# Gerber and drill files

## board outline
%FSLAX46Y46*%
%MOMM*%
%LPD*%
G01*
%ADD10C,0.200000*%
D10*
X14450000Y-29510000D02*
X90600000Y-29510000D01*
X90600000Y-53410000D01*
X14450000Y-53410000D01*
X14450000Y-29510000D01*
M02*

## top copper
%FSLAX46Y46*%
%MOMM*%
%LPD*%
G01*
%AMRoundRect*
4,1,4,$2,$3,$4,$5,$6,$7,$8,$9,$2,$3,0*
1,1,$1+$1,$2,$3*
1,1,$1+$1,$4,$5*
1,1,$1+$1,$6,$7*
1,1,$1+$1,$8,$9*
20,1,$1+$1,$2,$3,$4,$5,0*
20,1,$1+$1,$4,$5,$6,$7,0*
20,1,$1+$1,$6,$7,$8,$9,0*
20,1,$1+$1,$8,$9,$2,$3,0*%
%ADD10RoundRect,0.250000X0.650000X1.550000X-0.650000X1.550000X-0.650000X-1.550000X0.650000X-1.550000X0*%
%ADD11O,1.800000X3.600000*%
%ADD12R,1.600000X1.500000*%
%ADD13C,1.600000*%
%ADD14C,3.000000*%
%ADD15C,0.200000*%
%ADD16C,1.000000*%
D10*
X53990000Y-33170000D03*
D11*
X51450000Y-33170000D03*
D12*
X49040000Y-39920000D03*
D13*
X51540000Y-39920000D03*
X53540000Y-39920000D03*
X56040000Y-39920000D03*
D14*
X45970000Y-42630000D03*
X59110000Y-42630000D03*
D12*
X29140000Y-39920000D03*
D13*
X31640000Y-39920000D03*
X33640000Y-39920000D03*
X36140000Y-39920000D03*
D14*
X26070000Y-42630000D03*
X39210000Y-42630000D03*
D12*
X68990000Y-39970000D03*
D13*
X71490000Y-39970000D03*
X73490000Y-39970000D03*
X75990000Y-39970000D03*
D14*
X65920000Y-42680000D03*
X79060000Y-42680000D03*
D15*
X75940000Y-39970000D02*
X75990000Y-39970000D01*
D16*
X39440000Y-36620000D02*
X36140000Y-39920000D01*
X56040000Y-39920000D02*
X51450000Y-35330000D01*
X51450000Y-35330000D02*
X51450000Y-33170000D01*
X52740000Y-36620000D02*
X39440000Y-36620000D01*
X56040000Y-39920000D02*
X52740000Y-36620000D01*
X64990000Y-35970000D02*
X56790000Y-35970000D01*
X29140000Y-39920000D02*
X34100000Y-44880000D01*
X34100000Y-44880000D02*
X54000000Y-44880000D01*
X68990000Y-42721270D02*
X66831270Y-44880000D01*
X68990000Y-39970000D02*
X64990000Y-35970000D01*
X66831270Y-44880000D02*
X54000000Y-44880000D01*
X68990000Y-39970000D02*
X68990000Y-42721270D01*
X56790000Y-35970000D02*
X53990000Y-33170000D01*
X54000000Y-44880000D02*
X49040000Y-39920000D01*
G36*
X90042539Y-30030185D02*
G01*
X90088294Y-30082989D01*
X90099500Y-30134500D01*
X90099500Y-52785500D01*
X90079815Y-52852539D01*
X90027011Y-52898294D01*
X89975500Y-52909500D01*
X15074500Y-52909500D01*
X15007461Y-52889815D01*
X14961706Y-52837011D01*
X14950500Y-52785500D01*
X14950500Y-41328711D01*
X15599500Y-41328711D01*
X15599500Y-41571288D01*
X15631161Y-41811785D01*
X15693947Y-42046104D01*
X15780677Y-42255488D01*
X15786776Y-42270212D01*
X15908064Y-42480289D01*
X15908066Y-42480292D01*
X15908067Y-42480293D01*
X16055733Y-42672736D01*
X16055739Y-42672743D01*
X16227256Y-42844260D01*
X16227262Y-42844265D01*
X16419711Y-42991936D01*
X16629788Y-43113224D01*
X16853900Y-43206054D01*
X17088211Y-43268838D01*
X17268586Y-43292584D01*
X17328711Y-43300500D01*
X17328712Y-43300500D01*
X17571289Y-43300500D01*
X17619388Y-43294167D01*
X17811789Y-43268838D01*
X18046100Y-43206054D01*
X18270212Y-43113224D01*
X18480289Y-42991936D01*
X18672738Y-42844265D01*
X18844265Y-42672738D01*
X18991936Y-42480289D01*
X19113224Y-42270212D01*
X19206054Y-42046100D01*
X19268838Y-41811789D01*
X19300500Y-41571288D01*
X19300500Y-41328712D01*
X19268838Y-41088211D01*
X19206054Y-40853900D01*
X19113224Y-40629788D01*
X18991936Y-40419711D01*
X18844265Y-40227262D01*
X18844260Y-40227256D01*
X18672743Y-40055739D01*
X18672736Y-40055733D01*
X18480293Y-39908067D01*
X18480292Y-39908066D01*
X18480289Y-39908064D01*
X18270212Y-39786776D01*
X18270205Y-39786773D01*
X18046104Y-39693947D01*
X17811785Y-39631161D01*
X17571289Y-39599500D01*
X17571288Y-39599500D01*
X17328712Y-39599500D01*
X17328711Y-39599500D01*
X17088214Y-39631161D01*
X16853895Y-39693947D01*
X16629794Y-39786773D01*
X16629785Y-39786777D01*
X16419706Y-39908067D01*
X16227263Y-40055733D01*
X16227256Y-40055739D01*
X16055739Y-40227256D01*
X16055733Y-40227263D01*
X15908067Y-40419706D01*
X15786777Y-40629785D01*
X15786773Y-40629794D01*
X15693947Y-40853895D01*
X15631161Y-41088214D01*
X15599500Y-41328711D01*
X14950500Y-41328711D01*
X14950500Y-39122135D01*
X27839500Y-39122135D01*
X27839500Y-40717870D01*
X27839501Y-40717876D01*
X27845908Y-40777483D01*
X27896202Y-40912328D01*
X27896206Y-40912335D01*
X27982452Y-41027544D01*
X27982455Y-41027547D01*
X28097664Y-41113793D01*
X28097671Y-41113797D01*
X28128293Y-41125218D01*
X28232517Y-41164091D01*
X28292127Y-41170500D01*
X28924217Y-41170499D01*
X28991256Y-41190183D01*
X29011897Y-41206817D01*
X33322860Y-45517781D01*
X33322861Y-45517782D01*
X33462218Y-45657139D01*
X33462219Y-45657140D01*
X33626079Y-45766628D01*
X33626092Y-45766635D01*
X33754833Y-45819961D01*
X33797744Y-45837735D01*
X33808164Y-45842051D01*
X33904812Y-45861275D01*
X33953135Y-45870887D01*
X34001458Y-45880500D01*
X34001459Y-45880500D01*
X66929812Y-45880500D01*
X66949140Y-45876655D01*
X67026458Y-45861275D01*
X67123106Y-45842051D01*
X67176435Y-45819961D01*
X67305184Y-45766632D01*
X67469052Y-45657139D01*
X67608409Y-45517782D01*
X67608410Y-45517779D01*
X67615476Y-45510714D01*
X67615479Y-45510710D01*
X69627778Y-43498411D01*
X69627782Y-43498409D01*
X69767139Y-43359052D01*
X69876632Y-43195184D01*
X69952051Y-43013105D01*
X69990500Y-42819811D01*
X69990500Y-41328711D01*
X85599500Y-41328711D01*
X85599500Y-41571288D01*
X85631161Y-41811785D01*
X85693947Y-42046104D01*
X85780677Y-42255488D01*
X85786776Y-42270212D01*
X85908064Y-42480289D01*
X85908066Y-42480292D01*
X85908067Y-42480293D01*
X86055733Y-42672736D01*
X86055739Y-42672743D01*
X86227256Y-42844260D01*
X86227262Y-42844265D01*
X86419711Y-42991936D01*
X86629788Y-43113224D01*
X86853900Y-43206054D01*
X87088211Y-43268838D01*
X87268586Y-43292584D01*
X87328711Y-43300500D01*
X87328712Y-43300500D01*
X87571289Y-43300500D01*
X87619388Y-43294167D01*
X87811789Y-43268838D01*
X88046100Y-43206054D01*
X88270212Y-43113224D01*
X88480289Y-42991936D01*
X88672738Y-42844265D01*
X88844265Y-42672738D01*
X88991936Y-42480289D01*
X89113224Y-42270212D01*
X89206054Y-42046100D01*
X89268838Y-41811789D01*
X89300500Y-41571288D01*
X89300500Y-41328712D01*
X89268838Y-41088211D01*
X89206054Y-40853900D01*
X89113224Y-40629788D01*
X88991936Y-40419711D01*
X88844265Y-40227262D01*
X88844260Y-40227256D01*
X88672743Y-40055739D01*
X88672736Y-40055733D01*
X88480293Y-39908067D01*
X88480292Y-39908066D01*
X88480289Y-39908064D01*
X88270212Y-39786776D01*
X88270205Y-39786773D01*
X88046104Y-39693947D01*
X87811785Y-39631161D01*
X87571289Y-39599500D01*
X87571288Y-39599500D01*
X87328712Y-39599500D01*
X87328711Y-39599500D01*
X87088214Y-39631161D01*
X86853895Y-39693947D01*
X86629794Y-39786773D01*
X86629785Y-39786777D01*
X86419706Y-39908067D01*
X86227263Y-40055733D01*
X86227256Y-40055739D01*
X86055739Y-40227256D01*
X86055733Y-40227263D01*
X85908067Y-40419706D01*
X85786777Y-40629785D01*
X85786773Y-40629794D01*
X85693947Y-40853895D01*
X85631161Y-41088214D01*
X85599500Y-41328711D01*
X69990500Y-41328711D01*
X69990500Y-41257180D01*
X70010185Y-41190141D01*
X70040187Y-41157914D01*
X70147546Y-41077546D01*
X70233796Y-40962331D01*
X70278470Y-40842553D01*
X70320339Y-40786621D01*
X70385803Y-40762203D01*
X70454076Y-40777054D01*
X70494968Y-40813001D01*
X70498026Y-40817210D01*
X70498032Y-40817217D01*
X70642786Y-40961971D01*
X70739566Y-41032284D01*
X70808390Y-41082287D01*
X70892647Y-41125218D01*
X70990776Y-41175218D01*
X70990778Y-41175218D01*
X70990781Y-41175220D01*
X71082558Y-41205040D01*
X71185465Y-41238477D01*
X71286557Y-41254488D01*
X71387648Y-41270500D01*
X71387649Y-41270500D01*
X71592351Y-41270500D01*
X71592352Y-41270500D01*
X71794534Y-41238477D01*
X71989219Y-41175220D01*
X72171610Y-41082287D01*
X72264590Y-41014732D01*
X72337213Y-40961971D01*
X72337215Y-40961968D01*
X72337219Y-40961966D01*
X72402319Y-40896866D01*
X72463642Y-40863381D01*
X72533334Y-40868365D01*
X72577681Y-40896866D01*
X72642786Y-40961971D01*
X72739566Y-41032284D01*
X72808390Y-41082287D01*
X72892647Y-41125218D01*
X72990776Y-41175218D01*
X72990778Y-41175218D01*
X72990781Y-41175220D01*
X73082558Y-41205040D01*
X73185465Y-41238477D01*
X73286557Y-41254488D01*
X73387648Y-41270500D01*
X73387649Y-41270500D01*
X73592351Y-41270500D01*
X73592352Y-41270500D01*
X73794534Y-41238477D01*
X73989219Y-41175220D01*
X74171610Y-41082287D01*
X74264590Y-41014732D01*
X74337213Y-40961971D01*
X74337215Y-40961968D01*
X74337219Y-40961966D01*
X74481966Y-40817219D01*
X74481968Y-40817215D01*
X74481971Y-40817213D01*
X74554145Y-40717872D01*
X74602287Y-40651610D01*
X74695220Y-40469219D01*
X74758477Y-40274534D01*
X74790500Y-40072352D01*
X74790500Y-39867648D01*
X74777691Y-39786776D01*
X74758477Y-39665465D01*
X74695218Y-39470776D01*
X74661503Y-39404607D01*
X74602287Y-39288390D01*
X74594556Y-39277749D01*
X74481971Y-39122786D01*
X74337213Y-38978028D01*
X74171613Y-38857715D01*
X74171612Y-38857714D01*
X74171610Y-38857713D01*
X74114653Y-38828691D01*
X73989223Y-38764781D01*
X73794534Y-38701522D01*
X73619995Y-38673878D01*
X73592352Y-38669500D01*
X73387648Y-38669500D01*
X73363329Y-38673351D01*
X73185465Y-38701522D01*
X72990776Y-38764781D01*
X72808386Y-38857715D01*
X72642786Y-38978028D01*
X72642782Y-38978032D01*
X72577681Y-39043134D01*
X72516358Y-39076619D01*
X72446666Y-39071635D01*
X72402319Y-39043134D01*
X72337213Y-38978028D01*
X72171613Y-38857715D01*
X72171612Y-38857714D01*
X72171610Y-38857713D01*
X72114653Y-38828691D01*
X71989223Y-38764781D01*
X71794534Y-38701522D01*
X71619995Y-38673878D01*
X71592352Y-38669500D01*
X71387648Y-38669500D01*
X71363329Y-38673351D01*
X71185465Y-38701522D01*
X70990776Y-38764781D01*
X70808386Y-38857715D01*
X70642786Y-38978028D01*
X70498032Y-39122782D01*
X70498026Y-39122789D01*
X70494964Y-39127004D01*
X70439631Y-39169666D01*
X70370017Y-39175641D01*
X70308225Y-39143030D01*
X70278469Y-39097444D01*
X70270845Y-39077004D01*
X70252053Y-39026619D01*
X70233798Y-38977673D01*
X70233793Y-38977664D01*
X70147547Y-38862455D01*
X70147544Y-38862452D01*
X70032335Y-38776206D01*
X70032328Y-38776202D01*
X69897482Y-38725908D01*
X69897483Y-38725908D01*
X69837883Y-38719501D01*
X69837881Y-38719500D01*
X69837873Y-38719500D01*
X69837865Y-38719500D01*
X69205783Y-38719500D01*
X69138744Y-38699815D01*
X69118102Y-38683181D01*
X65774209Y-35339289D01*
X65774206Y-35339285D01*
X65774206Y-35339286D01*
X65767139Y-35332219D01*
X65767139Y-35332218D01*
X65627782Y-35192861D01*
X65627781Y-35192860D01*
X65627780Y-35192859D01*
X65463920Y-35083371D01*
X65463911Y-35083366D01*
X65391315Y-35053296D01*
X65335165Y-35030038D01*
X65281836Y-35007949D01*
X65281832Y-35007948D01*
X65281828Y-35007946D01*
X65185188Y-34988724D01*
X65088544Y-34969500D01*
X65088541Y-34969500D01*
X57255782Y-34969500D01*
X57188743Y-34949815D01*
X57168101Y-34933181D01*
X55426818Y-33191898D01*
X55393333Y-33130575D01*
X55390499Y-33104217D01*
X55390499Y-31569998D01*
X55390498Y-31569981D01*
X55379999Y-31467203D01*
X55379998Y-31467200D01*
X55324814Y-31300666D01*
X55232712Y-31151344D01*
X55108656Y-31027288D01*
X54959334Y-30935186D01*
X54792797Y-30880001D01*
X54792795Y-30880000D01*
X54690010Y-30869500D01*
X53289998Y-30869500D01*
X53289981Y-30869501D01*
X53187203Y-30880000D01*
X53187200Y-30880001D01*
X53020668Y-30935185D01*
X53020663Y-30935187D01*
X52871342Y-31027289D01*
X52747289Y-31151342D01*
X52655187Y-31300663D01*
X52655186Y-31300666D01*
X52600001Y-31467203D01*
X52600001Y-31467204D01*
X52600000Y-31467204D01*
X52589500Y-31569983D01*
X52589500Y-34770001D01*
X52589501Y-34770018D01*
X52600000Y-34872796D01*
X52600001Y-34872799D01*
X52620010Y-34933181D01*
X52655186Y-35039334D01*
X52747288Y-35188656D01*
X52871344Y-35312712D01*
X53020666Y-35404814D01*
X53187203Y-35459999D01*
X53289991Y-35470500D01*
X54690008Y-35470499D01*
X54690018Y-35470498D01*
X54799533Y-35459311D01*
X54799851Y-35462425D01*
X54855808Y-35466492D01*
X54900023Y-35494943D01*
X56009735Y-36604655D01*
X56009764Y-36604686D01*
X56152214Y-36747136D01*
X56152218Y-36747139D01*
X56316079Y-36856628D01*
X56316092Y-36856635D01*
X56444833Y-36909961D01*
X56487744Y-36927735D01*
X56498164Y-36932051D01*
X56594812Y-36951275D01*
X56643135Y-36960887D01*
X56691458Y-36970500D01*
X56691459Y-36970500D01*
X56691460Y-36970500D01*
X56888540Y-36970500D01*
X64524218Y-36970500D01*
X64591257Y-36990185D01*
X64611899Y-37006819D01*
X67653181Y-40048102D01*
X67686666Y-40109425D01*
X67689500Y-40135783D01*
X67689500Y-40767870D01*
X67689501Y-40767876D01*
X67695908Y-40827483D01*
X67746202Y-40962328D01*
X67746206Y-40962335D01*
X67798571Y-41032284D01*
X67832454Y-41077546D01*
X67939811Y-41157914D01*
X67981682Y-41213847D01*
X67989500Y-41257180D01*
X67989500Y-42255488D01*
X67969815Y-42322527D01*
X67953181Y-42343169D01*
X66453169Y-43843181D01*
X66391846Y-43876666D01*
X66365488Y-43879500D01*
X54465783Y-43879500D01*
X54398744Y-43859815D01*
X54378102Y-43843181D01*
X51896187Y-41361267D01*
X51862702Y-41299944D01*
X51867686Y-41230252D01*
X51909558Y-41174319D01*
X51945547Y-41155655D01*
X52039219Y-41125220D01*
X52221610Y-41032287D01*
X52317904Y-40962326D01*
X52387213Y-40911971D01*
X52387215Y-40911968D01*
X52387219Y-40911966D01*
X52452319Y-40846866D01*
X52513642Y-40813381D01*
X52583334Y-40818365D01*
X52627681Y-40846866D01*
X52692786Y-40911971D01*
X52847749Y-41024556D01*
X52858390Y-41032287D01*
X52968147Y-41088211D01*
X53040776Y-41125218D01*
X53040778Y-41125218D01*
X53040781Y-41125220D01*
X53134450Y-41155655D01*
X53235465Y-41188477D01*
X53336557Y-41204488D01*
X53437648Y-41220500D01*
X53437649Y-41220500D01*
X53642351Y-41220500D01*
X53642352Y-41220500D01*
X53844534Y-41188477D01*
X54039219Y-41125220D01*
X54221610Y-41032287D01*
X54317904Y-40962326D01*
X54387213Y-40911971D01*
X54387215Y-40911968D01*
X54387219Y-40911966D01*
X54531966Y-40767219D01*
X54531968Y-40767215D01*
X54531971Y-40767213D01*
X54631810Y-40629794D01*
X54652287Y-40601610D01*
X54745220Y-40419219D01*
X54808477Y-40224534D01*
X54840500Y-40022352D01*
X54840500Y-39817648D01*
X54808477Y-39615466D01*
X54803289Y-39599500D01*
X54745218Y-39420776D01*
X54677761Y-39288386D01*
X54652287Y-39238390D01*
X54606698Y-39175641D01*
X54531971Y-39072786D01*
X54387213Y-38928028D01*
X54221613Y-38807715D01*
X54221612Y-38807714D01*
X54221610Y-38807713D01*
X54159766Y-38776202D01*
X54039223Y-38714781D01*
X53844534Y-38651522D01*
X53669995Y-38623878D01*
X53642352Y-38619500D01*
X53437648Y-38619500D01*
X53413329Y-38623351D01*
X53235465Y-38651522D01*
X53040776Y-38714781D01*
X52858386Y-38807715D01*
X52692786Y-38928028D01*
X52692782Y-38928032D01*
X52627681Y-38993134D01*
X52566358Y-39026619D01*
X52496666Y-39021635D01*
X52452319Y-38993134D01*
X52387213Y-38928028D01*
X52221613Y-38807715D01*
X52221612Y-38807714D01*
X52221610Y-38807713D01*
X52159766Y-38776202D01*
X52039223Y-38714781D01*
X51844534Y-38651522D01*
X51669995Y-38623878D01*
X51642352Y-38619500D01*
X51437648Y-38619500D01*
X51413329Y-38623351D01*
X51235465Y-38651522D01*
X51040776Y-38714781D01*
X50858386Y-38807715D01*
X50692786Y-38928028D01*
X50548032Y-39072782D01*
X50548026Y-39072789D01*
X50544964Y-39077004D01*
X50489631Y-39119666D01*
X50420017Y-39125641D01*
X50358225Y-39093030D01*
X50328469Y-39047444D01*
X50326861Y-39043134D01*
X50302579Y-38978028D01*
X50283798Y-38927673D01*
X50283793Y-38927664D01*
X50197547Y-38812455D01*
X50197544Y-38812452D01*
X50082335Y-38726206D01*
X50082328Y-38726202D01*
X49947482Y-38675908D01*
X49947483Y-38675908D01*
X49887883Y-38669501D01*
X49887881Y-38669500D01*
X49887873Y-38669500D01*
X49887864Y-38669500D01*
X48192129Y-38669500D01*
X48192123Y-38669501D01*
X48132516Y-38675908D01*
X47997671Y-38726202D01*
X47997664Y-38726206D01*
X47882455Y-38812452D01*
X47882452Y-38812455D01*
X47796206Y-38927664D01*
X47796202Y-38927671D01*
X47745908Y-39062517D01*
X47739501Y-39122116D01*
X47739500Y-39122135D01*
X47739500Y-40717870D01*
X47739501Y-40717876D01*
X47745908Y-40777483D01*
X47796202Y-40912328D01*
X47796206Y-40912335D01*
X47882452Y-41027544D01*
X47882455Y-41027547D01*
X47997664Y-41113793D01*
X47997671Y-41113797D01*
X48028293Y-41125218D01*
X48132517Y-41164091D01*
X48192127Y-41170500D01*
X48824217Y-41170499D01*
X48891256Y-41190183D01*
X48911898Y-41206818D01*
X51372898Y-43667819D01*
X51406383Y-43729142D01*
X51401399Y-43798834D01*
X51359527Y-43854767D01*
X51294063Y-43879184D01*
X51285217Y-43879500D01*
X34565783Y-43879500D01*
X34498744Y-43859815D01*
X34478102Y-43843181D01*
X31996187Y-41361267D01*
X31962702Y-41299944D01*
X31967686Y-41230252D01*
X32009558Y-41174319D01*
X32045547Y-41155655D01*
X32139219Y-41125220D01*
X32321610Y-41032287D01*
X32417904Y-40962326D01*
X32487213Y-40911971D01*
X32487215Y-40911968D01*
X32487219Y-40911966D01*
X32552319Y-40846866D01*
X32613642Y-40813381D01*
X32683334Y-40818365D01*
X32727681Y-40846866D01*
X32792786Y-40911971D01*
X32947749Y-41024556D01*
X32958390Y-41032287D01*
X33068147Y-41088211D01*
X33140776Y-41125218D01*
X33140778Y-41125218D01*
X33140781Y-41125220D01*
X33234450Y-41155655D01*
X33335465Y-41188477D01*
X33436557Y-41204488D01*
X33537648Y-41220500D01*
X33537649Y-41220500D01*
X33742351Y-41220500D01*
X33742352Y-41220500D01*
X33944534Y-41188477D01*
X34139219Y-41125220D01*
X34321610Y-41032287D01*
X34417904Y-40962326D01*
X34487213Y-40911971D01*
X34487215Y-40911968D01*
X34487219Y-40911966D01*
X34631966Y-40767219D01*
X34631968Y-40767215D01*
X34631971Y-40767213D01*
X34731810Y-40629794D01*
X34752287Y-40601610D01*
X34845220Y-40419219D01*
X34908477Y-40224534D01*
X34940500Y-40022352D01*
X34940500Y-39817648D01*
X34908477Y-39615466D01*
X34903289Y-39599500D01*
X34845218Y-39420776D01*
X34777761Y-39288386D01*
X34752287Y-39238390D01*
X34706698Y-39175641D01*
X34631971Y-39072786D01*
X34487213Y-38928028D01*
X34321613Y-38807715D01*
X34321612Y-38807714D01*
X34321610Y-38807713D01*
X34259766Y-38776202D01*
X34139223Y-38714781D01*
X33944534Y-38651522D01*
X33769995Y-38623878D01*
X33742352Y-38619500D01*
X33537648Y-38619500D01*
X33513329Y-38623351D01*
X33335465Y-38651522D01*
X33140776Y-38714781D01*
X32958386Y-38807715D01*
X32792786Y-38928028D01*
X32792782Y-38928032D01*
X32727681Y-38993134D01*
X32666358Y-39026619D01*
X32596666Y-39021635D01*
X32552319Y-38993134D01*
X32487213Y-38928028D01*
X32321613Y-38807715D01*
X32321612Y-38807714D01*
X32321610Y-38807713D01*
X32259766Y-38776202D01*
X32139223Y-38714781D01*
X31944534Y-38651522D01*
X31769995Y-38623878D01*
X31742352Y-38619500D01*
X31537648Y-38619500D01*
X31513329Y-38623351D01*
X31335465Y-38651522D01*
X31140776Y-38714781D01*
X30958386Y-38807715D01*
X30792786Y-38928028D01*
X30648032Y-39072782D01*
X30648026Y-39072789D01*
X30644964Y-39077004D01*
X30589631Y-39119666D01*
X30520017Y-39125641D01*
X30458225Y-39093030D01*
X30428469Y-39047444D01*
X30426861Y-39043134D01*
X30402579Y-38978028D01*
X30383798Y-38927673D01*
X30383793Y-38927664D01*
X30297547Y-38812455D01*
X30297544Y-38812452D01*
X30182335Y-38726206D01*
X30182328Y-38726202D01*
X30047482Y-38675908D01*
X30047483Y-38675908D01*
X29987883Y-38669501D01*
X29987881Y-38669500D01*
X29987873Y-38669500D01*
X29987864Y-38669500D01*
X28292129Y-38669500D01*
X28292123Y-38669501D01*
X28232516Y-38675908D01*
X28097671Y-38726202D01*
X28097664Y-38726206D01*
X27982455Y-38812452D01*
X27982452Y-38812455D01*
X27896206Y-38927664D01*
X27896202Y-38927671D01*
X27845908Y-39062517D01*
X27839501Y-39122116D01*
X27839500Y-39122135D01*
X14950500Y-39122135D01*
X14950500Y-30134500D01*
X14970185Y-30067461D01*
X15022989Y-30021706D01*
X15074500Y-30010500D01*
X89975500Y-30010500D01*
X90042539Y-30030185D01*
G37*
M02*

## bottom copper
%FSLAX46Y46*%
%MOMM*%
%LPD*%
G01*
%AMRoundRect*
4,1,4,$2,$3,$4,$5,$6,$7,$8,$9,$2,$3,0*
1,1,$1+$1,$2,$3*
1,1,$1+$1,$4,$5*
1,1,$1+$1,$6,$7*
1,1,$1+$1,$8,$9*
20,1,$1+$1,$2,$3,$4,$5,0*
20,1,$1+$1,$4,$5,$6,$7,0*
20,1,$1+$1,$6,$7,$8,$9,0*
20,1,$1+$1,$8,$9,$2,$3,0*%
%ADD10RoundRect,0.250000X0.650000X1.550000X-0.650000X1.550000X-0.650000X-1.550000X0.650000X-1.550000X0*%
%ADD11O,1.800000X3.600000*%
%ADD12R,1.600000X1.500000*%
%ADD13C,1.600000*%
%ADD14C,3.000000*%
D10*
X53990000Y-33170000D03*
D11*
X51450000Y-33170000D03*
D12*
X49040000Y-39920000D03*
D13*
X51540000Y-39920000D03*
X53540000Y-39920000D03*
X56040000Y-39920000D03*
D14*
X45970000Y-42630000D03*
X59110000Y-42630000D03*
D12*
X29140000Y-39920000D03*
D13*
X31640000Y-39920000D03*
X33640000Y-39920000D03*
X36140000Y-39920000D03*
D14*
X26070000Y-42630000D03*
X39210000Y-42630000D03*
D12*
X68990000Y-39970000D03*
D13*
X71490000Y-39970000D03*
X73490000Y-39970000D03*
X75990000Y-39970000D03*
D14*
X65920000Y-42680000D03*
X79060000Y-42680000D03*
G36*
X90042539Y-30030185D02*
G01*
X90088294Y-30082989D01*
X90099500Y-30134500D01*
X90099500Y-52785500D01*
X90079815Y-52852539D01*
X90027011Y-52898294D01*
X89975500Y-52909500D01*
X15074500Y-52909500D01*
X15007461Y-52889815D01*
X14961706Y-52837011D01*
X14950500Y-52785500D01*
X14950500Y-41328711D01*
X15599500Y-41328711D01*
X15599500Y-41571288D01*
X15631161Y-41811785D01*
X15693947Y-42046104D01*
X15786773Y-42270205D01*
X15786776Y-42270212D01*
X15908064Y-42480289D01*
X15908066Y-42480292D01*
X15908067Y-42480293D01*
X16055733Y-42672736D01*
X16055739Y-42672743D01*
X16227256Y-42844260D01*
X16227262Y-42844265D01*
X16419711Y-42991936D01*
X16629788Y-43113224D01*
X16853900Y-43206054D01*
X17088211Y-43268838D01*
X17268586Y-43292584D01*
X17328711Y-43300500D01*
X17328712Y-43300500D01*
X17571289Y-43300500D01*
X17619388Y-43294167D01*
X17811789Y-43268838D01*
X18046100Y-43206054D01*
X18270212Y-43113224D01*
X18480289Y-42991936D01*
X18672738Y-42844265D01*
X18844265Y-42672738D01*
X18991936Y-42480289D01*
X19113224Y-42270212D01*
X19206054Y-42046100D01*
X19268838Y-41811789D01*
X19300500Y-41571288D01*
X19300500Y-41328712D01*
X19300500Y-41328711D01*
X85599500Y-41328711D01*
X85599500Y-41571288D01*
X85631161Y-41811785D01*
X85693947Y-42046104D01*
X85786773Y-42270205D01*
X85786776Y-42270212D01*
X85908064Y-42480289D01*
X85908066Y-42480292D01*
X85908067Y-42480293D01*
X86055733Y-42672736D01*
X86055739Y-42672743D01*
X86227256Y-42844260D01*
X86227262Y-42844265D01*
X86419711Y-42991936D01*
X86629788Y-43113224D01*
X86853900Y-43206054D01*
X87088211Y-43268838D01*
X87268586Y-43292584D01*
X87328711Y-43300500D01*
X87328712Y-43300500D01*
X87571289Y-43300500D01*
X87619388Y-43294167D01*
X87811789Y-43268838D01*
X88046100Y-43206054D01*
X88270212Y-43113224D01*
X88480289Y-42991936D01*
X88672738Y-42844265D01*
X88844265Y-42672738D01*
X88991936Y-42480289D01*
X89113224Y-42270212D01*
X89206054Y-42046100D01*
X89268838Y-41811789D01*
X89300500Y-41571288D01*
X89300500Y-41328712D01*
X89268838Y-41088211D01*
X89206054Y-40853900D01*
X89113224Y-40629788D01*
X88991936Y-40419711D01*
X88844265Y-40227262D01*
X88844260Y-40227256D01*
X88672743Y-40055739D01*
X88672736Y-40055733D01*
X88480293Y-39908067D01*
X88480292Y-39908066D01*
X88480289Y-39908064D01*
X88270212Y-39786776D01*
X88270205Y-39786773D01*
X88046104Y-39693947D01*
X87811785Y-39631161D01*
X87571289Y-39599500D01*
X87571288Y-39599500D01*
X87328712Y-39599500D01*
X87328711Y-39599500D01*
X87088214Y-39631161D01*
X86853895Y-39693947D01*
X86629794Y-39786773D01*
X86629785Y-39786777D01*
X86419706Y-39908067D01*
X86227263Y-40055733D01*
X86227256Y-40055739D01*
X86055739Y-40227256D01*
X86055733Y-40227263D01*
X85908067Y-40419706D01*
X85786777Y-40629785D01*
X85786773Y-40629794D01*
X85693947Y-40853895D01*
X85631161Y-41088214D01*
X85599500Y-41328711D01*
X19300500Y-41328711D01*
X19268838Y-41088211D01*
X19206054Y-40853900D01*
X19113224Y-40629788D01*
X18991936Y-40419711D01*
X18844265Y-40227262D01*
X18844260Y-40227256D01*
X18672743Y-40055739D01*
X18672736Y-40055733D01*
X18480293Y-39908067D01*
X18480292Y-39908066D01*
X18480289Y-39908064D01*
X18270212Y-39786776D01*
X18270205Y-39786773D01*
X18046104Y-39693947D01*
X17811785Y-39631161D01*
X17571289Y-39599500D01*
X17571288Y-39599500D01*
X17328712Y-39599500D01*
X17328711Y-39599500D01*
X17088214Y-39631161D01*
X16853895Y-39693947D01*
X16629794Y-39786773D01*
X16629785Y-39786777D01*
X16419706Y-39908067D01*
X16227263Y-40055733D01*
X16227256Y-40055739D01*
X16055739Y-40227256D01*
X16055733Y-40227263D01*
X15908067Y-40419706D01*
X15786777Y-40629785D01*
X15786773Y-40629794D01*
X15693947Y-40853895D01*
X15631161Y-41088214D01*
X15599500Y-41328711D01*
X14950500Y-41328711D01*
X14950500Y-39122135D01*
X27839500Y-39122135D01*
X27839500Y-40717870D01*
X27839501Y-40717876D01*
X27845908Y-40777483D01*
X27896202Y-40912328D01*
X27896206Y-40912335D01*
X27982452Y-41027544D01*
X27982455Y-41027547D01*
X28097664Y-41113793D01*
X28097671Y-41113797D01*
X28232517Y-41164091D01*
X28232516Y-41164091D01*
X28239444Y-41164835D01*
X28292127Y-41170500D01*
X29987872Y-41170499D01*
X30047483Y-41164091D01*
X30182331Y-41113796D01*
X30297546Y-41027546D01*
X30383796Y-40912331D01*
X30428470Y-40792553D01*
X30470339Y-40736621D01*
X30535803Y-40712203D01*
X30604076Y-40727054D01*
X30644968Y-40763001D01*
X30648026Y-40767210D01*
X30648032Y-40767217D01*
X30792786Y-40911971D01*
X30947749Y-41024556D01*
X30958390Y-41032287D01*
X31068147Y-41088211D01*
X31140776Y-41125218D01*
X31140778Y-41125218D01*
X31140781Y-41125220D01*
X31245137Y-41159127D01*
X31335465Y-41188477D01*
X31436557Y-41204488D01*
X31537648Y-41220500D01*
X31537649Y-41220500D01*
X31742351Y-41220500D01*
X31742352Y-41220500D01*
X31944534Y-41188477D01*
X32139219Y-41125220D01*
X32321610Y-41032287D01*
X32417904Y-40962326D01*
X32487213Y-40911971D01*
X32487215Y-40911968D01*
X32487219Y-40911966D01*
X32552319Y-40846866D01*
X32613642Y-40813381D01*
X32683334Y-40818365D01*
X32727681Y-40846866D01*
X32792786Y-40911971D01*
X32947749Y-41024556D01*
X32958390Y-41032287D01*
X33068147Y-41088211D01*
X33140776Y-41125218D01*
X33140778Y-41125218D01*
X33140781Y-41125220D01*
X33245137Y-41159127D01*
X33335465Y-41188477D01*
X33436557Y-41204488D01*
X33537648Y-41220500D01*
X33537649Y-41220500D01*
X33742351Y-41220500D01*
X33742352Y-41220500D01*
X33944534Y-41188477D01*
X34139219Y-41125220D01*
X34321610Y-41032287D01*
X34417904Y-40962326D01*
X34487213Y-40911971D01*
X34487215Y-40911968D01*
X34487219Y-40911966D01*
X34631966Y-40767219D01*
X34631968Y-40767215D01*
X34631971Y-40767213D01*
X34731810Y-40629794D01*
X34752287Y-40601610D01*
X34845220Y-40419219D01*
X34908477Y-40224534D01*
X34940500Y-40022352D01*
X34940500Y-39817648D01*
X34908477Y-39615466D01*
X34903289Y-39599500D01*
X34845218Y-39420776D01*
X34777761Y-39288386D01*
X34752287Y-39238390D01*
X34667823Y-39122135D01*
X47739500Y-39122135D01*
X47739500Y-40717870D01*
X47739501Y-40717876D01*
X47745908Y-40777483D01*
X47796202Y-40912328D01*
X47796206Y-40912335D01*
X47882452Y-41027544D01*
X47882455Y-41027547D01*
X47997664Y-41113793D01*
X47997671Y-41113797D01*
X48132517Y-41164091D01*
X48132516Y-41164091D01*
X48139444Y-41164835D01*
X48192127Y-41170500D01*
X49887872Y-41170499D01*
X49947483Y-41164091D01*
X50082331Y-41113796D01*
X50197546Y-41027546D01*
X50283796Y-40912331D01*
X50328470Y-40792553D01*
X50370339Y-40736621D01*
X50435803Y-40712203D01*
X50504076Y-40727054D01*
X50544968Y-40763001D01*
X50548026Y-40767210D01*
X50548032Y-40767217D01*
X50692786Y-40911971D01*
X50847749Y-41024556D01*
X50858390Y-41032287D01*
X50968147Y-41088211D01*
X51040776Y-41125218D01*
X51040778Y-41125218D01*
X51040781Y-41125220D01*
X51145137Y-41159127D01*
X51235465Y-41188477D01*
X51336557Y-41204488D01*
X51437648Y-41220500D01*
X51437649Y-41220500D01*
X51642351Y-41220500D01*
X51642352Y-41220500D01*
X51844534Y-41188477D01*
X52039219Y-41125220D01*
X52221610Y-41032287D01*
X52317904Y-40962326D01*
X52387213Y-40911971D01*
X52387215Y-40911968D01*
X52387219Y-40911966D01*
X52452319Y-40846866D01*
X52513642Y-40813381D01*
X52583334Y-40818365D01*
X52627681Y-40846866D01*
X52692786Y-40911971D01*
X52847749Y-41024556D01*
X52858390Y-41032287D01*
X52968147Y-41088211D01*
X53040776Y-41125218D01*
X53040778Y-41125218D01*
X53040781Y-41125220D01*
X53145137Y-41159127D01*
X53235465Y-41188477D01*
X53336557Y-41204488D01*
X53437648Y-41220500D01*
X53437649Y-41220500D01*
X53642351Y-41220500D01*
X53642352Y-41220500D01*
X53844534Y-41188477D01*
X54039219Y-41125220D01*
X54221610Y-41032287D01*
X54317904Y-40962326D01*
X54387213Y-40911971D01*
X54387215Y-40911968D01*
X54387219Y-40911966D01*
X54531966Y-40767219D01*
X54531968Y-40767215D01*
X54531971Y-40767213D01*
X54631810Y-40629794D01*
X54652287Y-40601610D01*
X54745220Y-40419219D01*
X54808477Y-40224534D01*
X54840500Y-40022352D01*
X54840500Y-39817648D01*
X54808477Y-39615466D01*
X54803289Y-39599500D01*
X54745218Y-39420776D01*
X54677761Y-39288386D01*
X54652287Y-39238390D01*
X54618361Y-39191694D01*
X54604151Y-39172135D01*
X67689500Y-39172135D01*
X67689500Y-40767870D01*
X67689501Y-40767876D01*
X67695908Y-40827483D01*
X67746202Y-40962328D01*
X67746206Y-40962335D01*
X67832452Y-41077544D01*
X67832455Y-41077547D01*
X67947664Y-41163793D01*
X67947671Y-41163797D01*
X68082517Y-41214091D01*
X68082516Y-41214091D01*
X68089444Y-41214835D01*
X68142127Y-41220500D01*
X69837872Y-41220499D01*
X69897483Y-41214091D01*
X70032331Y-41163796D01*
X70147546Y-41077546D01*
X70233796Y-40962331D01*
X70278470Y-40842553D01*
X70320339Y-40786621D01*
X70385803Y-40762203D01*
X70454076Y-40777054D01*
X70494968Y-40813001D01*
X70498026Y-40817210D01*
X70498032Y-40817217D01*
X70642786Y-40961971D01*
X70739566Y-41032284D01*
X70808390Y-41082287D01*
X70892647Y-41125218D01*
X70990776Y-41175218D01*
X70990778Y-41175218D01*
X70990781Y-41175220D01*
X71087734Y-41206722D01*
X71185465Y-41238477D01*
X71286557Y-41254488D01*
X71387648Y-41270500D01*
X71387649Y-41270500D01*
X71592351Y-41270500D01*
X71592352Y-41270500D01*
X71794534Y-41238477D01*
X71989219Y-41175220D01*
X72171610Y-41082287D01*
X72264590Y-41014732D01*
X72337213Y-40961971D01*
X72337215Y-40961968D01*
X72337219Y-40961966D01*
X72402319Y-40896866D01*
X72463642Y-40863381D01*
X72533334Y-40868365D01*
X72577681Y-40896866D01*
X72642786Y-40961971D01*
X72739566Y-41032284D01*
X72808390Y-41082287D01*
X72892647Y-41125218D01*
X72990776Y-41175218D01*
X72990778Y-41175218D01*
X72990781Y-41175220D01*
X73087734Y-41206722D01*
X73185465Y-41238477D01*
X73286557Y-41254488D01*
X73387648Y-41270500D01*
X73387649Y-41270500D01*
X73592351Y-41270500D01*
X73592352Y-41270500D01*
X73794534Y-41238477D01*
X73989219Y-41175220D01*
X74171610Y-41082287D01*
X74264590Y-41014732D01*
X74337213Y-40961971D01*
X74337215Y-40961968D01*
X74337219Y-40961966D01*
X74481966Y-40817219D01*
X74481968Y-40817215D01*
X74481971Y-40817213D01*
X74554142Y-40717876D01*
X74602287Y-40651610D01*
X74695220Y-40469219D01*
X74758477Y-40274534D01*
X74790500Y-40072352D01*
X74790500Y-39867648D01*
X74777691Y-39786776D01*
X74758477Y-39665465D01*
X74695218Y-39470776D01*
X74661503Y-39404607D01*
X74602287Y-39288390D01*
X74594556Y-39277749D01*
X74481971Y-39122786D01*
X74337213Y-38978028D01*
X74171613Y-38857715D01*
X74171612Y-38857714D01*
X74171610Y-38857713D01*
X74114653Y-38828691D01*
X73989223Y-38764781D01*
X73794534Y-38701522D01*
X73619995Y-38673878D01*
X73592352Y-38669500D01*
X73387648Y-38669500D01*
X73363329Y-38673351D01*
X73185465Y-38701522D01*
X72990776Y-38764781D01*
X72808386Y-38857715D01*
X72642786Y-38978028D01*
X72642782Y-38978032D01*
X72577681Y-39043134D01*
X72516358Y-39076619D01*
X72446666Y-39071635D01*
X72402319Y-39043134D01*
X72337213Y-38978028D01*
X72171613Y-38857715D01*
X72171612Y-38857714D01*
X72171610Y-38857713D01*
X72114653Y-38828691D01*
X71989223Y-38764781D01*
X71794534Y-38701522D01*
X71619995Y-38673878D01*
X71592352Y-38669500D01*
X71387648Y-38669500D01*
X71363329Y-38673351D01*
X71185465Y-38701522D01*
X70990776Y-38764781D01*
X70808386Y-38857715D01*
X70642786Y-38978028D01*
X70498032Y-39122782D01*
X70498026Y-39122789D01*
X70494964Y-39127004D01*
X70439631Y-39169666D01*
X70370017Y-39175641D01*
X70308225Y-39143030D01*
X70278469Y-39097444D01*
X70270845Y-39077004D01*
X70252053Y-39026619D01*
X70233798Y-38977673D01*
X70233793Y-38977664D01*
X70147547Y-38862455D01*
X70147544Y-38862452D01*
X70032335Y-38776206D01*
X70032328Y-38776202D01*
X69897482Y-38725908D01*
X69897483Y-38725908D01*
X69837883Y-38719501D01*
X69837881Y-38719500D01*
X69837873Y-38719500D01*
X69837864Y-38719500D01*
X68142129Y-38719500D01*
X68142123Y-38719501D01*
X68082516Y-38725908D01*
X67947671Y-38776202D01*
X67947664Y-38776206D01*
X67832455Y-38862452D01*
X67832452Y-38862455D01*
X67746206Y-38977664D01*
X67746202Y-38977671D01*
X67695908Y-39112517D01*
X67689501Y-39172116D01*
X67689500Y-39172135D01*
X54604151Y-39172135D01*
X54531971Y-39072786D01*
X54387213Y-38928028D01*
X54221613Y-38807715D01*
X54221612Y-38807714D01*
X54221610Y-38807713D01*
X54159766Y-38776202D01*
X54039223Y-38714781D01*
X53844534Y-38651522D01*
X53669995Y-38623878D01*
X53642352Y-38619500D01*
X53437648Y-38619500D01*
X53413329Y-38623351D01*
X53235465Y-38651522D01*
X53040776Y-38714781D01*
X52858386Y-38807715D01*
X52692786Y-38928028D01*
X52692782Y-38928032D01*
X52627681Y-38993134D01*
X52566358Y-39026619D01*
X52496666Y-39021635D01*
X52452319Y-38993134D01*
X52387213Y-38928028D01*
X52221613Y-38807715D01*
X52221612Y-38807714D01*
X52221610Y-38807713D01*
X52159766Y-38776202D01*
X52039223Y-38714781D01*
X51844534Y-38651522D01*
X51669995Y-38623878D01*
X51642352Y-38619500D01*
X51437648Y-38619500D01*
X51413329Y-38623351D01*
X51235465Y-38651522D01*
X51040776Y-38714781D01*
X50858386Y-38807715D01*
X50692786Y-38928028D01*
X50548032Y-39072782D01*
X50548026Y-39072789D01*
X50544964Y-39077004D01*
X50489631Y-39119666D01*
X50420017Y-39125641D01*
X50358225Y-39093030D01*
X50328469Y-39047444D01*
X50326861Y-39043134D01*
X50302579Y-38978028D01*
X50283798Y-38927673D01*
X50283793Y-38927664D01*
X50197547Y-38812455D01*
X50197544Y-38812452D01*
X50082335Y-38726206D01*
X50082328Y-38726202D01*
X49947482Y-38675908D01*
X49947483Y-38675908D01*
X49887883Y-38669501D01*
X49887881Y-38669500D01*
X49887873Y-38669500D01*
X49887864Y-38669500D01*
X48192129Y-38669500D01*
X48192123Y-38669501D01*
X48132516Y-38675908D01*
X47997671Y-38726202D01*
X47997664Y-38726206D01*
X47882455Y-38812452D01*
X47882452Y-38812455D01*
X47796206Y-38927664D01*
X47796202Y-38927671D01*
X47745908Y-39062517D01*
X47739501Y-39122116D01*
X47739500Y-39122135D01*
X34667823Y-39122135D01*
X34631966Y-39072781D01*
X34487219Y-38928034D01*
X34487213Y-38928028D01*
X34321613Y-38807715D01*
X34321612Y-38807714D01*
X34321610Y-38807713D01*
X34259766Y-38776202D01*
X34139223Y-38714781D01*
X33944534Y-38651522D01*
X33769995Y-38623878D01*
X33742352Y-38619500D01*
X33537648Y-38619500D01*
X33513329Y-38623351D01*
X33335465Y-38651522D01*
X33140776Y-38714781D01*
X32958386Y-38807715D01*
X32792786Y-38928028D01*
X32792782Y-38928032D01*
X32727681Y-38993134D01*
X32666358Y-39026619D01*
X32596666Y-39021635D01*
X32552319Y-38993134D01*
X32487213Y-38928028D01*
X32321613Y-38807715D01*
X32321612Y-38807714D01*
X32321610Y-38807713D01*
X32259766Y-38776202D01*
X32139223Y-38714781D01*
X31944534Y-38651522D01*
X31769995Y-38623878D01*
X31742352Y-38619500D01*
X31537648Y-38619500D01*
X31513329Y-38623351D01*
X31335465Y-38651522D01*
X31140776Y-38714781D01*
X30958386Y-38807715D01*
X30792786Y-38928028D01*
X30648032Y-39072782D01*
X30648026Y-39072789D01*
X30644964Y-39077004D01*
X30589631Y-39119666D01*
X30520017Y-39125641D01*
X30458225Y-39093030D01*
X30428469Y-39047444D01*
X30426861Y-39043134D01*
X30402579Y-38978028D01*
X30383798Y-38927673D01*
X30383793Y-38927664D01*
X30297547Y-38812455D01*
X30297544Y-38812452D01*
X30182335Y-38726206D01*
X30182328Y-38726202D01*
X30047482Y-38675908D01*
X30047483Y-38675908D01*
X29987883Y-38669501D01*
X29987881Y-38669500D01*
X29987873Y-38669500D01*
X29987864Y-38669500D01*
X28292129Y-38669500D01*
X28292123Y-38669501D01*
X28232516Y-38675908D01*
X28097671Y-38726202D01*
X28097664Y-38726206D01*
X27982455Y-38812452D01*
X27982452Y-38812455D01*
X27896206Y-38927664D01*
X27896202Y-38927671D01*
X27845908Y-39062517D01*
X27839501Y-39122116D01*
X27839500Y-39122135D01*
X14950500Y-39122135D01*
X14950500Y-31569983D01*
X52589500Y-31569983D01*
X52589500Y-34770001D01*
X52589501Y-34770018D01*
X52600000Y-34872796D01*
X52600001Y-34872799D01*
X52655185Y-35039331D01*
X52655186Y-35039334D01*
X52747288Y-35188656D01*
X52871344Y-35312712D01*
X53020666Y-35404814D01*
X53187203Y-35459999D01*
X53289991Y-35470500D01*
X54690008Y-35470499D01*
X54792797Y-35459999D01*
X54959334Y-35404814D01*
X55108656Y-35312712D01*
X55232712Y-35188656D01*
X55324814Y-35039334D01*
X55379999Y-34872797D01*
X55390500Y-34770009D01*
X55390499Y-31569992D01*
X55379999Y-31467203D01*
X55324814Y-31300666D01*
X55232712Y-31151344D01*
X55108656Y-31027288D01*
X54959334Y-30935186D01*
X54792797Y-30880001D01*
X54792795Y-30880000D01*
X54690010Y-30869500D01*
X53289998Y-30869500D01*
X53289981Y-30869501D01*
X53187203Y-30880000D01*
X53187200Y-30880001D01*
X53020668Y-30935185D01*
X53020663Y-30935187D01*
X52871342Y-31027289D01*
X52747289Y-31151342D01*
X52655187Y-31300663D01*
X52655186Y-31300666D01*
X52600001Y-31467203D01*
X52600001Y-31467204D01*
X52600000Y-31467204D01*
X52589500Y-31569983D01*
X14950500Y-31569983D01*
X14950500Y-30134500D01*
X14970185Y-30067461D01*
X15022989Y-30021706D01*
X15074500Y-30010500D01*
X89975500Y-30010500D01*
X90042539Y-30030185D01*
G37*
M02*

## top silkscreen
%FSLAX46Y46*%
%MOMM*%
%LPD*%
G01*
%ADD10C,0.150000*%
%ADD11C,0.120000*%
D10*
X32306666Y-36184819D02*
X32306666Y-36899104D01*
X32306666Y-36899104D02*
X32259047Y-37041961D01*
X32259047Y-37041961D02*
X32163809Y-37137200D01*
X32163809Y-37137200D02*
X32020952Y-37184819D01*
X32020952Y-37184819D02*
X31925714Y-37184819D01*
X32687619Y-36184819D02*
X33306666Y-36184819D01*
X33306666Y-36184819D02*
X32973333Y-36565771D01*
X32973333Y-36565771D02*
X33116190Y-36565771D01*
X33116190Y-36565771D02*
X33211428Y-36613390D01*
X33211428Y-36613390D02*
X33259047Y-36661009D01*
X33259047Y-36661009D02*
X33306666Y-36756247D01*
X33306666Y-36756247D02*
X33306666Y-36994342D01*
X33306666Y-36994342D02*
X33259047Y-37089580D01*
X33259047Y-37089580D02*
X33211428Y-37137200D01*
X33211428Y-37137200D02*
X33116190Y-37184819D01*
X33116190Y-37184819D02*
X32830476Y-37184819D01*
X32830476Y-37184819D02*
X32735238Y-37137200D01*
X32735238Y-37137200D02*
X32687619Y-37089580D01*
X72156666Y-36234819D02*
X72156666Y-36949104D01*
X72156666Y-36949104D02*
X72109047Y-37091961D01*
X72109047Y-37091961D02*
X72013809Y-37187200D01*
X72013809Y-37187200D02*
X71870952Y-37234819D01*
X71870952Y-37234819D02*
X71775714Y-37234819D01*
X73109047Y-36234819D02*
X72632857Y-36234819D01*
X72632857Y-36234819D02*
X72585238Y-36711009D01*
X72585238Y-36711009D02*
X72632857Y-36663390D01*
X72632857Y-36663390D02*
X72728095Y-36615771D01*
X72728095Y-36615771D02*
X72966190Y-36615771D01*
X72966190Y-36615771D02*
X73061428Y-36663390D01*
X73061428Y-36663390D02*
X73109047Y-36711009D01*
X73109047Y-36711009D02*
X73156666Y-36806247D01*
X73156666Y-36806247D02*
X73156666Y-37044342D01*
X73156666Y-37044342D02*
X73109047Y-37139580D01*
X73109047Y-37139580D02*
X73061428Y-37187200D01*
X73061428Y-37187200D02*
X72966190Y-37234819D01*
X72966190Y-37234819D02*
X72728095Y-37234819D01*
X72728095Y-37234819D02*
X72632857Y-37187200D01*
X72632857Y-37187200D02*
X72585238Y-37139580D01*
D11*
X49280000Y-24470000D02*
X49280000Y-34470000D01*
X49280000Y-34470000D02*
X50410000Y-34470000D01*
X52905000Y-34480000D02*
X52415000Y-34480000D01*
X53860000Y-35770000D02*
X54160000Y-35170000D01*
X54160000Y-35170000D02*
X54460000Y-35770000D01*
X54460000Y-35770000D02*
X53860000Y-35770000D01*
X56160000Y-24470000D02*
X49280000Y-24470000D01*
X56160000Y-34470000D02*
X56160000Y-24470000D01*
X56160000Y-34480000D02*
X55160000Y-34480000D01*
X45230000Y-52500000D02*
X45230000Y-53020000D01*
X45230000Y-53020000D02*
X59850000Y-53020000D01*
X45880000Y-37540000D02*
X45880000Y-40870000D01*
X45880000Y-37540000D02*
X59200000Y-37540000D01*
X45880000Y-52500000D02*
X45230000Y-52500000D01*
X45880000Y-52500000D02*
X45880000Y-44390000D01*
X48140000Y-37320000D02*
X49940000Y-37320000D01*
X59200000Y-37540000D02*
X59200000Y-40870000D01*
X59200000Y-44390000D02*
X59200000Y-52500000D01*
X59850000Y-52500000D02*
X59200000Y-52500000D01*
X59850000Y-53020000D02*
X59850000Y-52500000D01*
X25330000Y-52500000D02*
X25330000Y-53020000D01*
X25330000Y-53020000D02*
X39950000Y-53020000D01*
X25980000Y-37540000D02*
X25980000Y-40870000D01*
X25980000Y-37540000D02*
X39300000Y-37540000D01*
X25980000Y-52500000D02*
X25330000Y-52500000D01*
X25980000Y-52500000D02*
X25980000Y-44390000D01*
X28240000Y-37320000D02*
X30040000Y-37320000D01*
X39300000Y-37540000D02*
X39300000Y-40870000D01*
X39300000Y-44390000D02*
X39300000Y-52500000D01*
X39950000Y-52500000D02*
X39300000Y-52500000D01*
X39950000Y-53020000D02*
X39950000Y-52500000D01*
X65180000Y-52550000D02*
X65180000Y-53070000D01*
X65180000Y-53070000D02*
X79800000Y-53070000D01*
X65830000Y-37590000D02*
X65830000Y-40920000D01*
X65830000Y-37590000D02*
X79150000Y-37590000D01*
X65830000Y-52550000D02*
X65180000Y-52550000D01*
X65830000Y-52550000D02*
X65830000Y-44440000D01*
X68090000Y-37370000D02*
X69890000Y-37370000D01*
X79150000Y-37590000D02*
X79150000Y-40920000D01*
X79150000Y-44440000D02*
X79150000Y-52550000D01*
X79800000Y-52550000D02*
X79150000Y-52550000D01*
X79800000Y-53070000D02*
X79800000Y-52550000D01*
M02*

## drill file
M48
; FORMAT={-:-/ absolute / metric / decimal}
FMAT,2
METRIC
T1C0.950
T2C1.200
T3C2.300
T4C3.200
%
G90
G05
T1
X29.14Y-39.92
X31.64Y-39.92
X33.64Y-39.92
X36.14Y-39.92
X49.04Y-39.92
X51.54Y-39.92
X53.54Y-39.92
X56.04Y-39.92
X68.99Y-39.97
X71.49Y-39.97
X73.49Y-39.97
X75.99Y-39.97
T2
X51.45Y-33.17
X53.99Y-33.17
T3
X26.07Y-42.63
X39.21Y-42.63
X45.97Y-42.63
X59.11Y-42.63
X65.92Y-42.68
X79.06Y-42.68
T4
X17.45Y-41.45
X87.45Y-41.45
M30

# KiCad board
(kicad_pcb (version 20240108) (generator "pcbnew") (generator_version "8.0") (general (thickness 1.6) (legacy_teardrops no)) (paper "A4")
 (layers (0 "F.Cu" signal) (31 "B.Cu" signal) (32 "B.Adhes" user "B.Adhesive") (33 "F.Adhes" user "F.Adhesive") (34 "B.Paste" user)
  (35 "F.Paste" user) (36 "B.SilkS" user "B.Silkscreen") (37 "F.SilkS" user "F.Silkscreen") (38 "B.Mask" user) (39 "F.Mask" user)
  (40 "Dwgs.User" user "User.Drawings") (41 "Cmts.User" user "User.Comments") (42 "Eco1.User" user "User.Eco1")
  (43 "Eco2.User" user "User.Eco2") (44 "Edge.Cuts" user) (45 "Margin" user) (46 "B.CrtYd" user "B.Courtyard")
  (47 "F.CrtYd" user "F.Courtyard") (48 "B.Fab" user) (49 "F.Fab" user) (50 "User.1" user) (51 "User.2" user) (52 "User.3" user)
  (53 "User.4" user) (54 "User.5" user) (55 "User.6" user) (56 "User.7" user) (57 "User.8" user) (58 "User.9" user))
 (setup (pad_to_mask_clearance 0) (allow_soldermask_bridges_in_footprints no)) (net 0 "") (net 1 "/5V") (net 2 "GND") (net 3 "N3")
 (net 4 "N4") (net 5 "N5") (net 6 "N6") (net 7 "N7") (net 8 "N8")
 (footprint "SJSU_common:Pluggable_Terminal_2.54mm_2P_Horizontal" (layer "F.Cu") (at 52.16 38.47 180)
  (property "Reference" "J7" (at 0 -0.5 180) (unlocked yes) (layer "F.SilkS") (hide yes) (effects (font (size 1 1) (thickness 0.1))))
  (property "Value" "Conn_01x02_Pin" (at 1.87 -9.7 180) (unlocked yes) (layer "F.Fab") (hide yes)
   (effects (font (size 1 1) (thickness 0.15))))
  (fp_line (start 2.88 14) (end 2.88 4) (stroke (width 0.12) (type solid)) (layer "F.SilkS"))
  (fp_line (start 2.88 4) (end 1.75 4) (stroke (width 0.12) (type solid)) (layer "F.SilkS"))
  (fp_line (start -0.745 3.99) (end -0.255 3.99) (stroke (width 0.12) (type solid)) (layer "F.SilkS"))
  (fp_line (start -1.7 2.7) (end -2 3.3) (stroke (width 0.12) (type solid)) (layer "F.SilkS"))
  (fp_line (start -2 3.3) (end -2.3 2.7) (stroke (width 0.12) (type solid)) (layer "F.SilkS"))
  (fp_line (start -2.3 2.7) (end -1.7 2.7) (stroke (width 0.12) (type solid)) (layer "F.SilkS"))
  (fp_line (start -4 14) (end 2.88 14) (stroke (width 0.12) (type solid)) (layer "F.SilkS"))
  (fp_line (start -4 4) (end -4 14) (stroke (width 0.12) (type solid)) (layer "F.SilkS"))
  (fp_line (start -4 3.99) (end -3 3.99) (stroke (width 0.12) (type solid)) (layer "F.SilkS"))
  (pad "1" thru_hole roundrect (at -1.83 5.3 180) (size 1.8 3.6) (drill 1.2) (layers "*.Cu" "*.Mask") (remove_unused_layers no)
   (roundrect_rratio 0.138889) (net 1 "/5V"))
  (pad "2" thru_hole oval (at 0.71 5.3 180) (size 1.8 3.6) (drill 1.2) (layers "*.Cu" "*.Mask") (remove_unused_layers no) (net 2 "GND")))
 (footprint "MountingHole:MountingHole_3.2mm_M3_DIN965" (layer "F.Cu") (at 17.45 41.45)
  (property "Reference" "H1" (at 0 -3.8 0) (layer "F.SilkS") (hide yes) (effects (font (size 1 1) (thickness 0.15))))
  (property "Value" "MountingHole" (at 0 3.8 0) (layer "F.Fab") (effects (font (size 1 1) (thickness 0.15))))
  (pad "" np_thru_hole circle (at 0 0) (size 3.2 3.2) (drill 3.2) (layers "*.Cu" "*.Mask")))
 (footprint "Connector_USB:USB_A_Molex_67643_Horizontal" (layer "F.Cu") (at 49.04 39.92)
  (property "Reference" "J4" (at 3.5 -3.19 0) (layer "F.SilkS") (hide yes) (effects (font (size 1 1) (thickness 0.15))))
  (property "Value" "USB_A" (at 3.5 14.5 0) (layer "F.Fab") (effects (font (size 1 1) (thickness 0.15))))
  (fp_line (start -3.81 12.58) (end -3.81 13.1) (stroke (width 0.12) (type solid)) (layer "F.SilkS"))
  (fp_line (start -3.81 13.1) (end 10.81 13.1) (stroke (width 0.12) (type solid)) (layer "F.SilkS"))
  (fp_line (start -3.16 -2.38) (end -3.16 0.95) (stroke (width 0.12) (type solid)) (layer "F.SilkS"))
  (fp_line (start -3.16 -2.38) (end 10.16 -2.38) (stroke (width 0.12) (type solid)) (layer "F.SilkS"))
  (fp_line (start -3.16 12.58) (end -3.81 12.58) (stroke (width 0.12) (type solid)) (layer "F.SilkS"))
  (fp_line (start -3.16 12.58) (end -3.16 4.47) (stroke (width 0.12) (type solid)) (layer "F.SilkS"))
  (fp_line (start -0.9 -2.6) (end 0.9 -2.6) (stroke (width 0.12) (type solid)) (layer "F.SilkS"))
  (fp_line (start 10.16 -2.38) (end 10.16 0.95) (stroke (width 0.12) (type solid)) (layer "F.SilkS"))
  (fp_line (start 10.16 4.47) (end 10.16 12.58) (stroke (width 0.12) (type solid)) (layer "F.SilkS"))
  (fp_line (start 10.81 12.58) (end 10.16 12.58) (stroke (width 0.12) (type solid)) (layer "F.SilkS"))
  (fp_line (start 10.81 13.1) (end 10.81 12.58) (stroke (width 0.12) (type solid)) (layer "F.SilkS"))
  (pad "1" thru_hole rect (at 0 0) (size 1.6 1.5) (drill 0.95) (layers "*.Cu" "*.Mask") (remove_unused_layers no) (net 1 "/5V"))
  (pad "2" thru_hole circle (at 2.5 0) (size 1.6 1.6) (drill 0.95) (layers "*.Cu" "*.Mask") (remove_unused_layers no) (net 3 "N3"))
  (pad "3" thru_hole circle (at 4.5 0) (size 1.6 1.6) (drill 0.95) (layers "*.Cu" "*.Mask") (remove_unused_layers no) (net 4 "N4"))
  (pad "4" thru_hole circle (at 7 0) (size 1.6 1.6) (drill 0.95) (layers "*.Cu" "*.Mask") (remove_unused_layers no) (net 2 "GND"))
  (pad "5" thru_hole circle (at -3.07 2.71) (size 3 3) (drill 2.3) (layers "*.Cu" "*.Mask") (remove_unused_layers no) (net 2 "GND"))
  (pad "5" thru_hole circle (at 10.07 2.71) (size 3 3) (drill 2.3) (layers "*.Cu" "*.Mask") (remove_unused_layers no) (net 2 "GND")))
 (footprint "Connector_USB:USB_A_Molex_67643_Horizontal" (layer "F.Cu") (at 29.14 39.92)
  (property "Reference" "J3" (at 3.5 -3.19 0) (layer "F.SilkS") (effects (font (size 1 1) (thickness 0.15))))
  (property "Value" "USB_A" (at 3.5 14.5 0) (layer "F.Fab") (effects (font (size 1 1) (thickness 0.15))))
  (fp_line (start -3.81 12.58) (end -3.81 13.1) (stroke (width 0.12) (type solid)) (layer "F.SilkS"))
  (fp_line (start -3.81 13.1) (end 10.81 13.1) (stroke (width 0.12) (type solid)) (layer "F.SilkS"))
  (fp_line (start -3.16 -2.38) (end -3.16 0.95) (stroke (width 0.12) (type solid)) (layer "F.SilkS"))
  (fp_line (start -3.16 -2.38) (end 10.16 -2.38) (stroke (width 0.12) (type solid)) (layer "F.SilkS"))
  (fp_line (start -3.16 12.58) (end -3.81 12.58) (stroke (width 0.12) (type solid)) (layer "F.SilkS"))
  (fp_line (start -3.16 12.58) (end -3.16 4.47) (stroke (width 0.12) (type solid)) (layer "F.SilkS"))
  (fp_line (start -0.9 -2.6) (end 0.9 -2.6) (stroke (width 0.12) (type solid)) (layer "F.SilkS"))
  (fp_line (start 10.16 -2.38) (end 10.16 0.95) (stroke (width 0.12) (type solid)) (layer "F.SilkS"))
  (fp_line (start 10.16 4.47) (end 10.16 12.58) (stroke (width 0.12) (type solid)) (layer "F.SilkS"))
  (fp_line (start 10.81 12.58) (end 10.16 12.58) (stroke (width 0.12) (type solid)) (layer "F.SilkS"))
  (fp_line (start 10.81 13.1) (end 10.81 12.58) (stroke (width 0.12) (type solid)) (layer "F.SilkS"))
  (pad "1" thru_hole rect (at 0 0) (size 1.6 1.5) (drill 0.95) (layers "*.Cu" "*.Mask") (remove_unused_layers no) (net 1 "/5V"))
  (pad "2" thru_hole circle (at 2.5 0) (size 1.6 1.6) (drill 0.95) (layers "*.Cu" "*.Mask") (remove_unused_layers no) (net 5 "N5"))
  (pad "3" thru_hole circle (at 4.5 0) (size 1.6 1.6) (drill 0.95) (layers "*.Cu" "*.Mask") (remove_unused_layers no) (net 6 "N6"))
  (pad "4" thru_hole circle (at 7 0) (size 1.6 1.6) (drill 0.95) (layers "*.Cu" "*.Mask") (remove_unused_layers no) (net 2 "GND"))
  (pad "5" thru_hole circle (at -3.07 2.71) (size 3 3) (drill 2.3) (layers "*.Cu" "*.Mask") (remove_unused_layers no) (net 2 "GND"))
  (pad "5" thru_hole circle (at 10.07 2.71) (size 3 3) (drill 2.3) (layers "*.Cu" "*.Mask") (remove_unused_layers no) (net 2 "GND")))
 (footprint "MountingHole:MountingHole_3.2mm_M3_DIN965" (layer "F.Cu") (at 87.45 41.45)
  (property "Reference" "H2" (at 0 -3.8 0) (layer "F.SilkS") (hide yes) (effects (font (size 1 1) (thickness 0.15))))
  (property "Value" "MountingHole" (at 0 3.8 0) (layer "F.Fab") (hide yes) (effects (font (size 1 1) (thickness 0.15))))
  (pad "" np_thru_hole circle (at 0 0) (size 3.2 3.2) (drill 3.2) (layers "*.Cu" "*.Mask")))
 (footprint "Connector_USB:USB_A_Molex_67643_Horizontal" (layer "F.Cu") (at 68.99 39.97)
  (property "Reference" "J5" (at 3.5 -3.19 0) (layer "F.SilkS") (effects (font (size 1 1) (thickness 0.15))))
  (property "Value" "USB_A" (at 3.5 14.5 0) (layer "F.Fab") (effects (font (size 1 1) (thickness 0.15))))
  (fp_line (start -3.81 12.58) (end -3.81 13.1) (stroke (width 0.12) (type solid)) (layer "F.SilkS"))
  (fp_line (start -3.81 13.1) (end 10.81 13.1) (stroke (width 0.12) (type solid)) (layer "F.SilkS"))
  (fp_line (start -3.16 -2.38) (end -3.16 0.95) (stroke (width 0.12) (type solid)) (layer "F.SilkS"))
  (fp_line (start -3.16 -2.38) (end 10.16 -2.38) (stroke (width 0.12) (type solid)) (layer "F.SilkS"))
  (fp_line (start -3.16 12.58) (end -3.81 12.58) (stroke (width 0.12) (type solid)) (layer "F.SilkS"))
  (fp_line (start -3.16 12.58) (end -3.16 4.47) (stroke (width 0.12) (type solid)) (layer "F.SilkS"))
  (fp_line (start -0.9 -2.6) (end 0.9 -2.6) (stroke (width 0.12) (type solid)) (layer "F.SilkS"))
  (fp_line (start 10.16 -2.38) (end 10.16 0.95) (stroke (width 0.12) (type solid)) (layer "F.SilkS"))
  (fp_line (start 10.16 4.47) (end 10.16 12.58) (stroke (width 0.12) (type solid)) (layer "F.SilkS"))
  (fp_line (start 10.81 12.58) (end 10.16 12.58) (stroke (width 0.12) (type solid)) (layer "F.SilkS"))
  (fp_line (start 10.81 13.1) (end 10.81 12.58) (stroke (width 0.12) (type solid)) (layer "F.SilkS"))
  (pad "1" thru_hole rect (at 0 0) (size 1.6 1.5) (drill 0.95) (layers "*.Cu" "*.Mask") (remove_unused_layers no) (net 1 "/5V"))
  (pad "2" thru_hole circle (at 2.5 0) (size 1.6 1.6) (drill 0.95) (layers "*.Cu" "*.Mask") (remove_unused_layers no) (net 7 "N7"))
  (pad "3" thru_hole circle (at 4.5 0) (size 1.6 1.6) (drill 0.95) (layers "*.Cu" "*.Mask") (remove_unused_layers no) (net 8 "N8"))
  (pad "4" thru_hole circle (at 7 0) (size 1.6 1.6) (drill 0.95) (layers "*.Cu" "*.Mask") (remove_unused_layers no) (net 2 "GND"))
  (pad "5" thru_hole circle (at -3.07 2.71) (size 3 3) (drill 2.3) (layers "*.Cu" "*.Mask") (remove_unused_layers no) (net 2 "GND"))
  (pad "5" thru_hole circle (at 10.07 2.71) (size 3 3) (drill 2.3) (layers "*.Cu" "*.Mask") (remove_unused_layers no) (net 2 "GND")))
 (gr_rect (start 14.45 29.51) (end 90.6 53.41) (stroke (width 0.2) (type default)) (fill none) (layer "Edge.Cuts"))
 (segment (start 75.94 39.97) (end 75.99 39.97) (width 0.2) (layer "F.Cu") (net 2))
 (segment (start 39.44 36.62) (end 36.14 39.92) (width 1) (layer "F.Cu") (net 2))
 (segment (start 56.04 39.92) (end 51.45 35.33) (width 1) (layer "F.Cu") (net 2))
 (segment (start 51.45 35.33) (end 51.45 33.17) (width 1) (layer "F.Cu") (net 2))
 (segment (start 52.74 36.62) (end 39.44 36.62) (width 1) (layer "F.Cu") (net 2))
 (segment (start 56.04 39.92) (end 52.74 36.62) (width 1) (layer "F.Cu") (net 2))
 (segment (start 64.99 35.97) (end 56.79 35.97) (width 1) (layer "F.Cu") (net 1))
 (segment (start 29.14 39.92) (end 34.1 44.88) (width 1) (layer "F.Cu") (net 1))
 (segment (start 34.1 44.88) (end 54 44.88) (width 1) (layer "F.Cu") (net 1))
 (segment (start 68.99 42.72127) (end 66.83127 44.88) (width 1) (layer "F.Cu") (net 1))
 (segment (start 68.99 39.97) (end 64.99 35.97) (width 1) (layer "F.Cu") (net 1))
 (segment (start 66.83127 44.88) (end 54 44.88) (width 1) (layer "F.Cu") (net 1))
 (segment (start 68.99 39.97) (end 68.99 42.72127) (width 1) (layer "F.Cu") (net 1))
 (segment (start 56.79 35.97) (end 53.99 33.17) (width 1) (layer "F.Cu") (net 1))
 (segment (start 54 44.88) (end 49.04 39.92) (width 1) (layer "F.Cu") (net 1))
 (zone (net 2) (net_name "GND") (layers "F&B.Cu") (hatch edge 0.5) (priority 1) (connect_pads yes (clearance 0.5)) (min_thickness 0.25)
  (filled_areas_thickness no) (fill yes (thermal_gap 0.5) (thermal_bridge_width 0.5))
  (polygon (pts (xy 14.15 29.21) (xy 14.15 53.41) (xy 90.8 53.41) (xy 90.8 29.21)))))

